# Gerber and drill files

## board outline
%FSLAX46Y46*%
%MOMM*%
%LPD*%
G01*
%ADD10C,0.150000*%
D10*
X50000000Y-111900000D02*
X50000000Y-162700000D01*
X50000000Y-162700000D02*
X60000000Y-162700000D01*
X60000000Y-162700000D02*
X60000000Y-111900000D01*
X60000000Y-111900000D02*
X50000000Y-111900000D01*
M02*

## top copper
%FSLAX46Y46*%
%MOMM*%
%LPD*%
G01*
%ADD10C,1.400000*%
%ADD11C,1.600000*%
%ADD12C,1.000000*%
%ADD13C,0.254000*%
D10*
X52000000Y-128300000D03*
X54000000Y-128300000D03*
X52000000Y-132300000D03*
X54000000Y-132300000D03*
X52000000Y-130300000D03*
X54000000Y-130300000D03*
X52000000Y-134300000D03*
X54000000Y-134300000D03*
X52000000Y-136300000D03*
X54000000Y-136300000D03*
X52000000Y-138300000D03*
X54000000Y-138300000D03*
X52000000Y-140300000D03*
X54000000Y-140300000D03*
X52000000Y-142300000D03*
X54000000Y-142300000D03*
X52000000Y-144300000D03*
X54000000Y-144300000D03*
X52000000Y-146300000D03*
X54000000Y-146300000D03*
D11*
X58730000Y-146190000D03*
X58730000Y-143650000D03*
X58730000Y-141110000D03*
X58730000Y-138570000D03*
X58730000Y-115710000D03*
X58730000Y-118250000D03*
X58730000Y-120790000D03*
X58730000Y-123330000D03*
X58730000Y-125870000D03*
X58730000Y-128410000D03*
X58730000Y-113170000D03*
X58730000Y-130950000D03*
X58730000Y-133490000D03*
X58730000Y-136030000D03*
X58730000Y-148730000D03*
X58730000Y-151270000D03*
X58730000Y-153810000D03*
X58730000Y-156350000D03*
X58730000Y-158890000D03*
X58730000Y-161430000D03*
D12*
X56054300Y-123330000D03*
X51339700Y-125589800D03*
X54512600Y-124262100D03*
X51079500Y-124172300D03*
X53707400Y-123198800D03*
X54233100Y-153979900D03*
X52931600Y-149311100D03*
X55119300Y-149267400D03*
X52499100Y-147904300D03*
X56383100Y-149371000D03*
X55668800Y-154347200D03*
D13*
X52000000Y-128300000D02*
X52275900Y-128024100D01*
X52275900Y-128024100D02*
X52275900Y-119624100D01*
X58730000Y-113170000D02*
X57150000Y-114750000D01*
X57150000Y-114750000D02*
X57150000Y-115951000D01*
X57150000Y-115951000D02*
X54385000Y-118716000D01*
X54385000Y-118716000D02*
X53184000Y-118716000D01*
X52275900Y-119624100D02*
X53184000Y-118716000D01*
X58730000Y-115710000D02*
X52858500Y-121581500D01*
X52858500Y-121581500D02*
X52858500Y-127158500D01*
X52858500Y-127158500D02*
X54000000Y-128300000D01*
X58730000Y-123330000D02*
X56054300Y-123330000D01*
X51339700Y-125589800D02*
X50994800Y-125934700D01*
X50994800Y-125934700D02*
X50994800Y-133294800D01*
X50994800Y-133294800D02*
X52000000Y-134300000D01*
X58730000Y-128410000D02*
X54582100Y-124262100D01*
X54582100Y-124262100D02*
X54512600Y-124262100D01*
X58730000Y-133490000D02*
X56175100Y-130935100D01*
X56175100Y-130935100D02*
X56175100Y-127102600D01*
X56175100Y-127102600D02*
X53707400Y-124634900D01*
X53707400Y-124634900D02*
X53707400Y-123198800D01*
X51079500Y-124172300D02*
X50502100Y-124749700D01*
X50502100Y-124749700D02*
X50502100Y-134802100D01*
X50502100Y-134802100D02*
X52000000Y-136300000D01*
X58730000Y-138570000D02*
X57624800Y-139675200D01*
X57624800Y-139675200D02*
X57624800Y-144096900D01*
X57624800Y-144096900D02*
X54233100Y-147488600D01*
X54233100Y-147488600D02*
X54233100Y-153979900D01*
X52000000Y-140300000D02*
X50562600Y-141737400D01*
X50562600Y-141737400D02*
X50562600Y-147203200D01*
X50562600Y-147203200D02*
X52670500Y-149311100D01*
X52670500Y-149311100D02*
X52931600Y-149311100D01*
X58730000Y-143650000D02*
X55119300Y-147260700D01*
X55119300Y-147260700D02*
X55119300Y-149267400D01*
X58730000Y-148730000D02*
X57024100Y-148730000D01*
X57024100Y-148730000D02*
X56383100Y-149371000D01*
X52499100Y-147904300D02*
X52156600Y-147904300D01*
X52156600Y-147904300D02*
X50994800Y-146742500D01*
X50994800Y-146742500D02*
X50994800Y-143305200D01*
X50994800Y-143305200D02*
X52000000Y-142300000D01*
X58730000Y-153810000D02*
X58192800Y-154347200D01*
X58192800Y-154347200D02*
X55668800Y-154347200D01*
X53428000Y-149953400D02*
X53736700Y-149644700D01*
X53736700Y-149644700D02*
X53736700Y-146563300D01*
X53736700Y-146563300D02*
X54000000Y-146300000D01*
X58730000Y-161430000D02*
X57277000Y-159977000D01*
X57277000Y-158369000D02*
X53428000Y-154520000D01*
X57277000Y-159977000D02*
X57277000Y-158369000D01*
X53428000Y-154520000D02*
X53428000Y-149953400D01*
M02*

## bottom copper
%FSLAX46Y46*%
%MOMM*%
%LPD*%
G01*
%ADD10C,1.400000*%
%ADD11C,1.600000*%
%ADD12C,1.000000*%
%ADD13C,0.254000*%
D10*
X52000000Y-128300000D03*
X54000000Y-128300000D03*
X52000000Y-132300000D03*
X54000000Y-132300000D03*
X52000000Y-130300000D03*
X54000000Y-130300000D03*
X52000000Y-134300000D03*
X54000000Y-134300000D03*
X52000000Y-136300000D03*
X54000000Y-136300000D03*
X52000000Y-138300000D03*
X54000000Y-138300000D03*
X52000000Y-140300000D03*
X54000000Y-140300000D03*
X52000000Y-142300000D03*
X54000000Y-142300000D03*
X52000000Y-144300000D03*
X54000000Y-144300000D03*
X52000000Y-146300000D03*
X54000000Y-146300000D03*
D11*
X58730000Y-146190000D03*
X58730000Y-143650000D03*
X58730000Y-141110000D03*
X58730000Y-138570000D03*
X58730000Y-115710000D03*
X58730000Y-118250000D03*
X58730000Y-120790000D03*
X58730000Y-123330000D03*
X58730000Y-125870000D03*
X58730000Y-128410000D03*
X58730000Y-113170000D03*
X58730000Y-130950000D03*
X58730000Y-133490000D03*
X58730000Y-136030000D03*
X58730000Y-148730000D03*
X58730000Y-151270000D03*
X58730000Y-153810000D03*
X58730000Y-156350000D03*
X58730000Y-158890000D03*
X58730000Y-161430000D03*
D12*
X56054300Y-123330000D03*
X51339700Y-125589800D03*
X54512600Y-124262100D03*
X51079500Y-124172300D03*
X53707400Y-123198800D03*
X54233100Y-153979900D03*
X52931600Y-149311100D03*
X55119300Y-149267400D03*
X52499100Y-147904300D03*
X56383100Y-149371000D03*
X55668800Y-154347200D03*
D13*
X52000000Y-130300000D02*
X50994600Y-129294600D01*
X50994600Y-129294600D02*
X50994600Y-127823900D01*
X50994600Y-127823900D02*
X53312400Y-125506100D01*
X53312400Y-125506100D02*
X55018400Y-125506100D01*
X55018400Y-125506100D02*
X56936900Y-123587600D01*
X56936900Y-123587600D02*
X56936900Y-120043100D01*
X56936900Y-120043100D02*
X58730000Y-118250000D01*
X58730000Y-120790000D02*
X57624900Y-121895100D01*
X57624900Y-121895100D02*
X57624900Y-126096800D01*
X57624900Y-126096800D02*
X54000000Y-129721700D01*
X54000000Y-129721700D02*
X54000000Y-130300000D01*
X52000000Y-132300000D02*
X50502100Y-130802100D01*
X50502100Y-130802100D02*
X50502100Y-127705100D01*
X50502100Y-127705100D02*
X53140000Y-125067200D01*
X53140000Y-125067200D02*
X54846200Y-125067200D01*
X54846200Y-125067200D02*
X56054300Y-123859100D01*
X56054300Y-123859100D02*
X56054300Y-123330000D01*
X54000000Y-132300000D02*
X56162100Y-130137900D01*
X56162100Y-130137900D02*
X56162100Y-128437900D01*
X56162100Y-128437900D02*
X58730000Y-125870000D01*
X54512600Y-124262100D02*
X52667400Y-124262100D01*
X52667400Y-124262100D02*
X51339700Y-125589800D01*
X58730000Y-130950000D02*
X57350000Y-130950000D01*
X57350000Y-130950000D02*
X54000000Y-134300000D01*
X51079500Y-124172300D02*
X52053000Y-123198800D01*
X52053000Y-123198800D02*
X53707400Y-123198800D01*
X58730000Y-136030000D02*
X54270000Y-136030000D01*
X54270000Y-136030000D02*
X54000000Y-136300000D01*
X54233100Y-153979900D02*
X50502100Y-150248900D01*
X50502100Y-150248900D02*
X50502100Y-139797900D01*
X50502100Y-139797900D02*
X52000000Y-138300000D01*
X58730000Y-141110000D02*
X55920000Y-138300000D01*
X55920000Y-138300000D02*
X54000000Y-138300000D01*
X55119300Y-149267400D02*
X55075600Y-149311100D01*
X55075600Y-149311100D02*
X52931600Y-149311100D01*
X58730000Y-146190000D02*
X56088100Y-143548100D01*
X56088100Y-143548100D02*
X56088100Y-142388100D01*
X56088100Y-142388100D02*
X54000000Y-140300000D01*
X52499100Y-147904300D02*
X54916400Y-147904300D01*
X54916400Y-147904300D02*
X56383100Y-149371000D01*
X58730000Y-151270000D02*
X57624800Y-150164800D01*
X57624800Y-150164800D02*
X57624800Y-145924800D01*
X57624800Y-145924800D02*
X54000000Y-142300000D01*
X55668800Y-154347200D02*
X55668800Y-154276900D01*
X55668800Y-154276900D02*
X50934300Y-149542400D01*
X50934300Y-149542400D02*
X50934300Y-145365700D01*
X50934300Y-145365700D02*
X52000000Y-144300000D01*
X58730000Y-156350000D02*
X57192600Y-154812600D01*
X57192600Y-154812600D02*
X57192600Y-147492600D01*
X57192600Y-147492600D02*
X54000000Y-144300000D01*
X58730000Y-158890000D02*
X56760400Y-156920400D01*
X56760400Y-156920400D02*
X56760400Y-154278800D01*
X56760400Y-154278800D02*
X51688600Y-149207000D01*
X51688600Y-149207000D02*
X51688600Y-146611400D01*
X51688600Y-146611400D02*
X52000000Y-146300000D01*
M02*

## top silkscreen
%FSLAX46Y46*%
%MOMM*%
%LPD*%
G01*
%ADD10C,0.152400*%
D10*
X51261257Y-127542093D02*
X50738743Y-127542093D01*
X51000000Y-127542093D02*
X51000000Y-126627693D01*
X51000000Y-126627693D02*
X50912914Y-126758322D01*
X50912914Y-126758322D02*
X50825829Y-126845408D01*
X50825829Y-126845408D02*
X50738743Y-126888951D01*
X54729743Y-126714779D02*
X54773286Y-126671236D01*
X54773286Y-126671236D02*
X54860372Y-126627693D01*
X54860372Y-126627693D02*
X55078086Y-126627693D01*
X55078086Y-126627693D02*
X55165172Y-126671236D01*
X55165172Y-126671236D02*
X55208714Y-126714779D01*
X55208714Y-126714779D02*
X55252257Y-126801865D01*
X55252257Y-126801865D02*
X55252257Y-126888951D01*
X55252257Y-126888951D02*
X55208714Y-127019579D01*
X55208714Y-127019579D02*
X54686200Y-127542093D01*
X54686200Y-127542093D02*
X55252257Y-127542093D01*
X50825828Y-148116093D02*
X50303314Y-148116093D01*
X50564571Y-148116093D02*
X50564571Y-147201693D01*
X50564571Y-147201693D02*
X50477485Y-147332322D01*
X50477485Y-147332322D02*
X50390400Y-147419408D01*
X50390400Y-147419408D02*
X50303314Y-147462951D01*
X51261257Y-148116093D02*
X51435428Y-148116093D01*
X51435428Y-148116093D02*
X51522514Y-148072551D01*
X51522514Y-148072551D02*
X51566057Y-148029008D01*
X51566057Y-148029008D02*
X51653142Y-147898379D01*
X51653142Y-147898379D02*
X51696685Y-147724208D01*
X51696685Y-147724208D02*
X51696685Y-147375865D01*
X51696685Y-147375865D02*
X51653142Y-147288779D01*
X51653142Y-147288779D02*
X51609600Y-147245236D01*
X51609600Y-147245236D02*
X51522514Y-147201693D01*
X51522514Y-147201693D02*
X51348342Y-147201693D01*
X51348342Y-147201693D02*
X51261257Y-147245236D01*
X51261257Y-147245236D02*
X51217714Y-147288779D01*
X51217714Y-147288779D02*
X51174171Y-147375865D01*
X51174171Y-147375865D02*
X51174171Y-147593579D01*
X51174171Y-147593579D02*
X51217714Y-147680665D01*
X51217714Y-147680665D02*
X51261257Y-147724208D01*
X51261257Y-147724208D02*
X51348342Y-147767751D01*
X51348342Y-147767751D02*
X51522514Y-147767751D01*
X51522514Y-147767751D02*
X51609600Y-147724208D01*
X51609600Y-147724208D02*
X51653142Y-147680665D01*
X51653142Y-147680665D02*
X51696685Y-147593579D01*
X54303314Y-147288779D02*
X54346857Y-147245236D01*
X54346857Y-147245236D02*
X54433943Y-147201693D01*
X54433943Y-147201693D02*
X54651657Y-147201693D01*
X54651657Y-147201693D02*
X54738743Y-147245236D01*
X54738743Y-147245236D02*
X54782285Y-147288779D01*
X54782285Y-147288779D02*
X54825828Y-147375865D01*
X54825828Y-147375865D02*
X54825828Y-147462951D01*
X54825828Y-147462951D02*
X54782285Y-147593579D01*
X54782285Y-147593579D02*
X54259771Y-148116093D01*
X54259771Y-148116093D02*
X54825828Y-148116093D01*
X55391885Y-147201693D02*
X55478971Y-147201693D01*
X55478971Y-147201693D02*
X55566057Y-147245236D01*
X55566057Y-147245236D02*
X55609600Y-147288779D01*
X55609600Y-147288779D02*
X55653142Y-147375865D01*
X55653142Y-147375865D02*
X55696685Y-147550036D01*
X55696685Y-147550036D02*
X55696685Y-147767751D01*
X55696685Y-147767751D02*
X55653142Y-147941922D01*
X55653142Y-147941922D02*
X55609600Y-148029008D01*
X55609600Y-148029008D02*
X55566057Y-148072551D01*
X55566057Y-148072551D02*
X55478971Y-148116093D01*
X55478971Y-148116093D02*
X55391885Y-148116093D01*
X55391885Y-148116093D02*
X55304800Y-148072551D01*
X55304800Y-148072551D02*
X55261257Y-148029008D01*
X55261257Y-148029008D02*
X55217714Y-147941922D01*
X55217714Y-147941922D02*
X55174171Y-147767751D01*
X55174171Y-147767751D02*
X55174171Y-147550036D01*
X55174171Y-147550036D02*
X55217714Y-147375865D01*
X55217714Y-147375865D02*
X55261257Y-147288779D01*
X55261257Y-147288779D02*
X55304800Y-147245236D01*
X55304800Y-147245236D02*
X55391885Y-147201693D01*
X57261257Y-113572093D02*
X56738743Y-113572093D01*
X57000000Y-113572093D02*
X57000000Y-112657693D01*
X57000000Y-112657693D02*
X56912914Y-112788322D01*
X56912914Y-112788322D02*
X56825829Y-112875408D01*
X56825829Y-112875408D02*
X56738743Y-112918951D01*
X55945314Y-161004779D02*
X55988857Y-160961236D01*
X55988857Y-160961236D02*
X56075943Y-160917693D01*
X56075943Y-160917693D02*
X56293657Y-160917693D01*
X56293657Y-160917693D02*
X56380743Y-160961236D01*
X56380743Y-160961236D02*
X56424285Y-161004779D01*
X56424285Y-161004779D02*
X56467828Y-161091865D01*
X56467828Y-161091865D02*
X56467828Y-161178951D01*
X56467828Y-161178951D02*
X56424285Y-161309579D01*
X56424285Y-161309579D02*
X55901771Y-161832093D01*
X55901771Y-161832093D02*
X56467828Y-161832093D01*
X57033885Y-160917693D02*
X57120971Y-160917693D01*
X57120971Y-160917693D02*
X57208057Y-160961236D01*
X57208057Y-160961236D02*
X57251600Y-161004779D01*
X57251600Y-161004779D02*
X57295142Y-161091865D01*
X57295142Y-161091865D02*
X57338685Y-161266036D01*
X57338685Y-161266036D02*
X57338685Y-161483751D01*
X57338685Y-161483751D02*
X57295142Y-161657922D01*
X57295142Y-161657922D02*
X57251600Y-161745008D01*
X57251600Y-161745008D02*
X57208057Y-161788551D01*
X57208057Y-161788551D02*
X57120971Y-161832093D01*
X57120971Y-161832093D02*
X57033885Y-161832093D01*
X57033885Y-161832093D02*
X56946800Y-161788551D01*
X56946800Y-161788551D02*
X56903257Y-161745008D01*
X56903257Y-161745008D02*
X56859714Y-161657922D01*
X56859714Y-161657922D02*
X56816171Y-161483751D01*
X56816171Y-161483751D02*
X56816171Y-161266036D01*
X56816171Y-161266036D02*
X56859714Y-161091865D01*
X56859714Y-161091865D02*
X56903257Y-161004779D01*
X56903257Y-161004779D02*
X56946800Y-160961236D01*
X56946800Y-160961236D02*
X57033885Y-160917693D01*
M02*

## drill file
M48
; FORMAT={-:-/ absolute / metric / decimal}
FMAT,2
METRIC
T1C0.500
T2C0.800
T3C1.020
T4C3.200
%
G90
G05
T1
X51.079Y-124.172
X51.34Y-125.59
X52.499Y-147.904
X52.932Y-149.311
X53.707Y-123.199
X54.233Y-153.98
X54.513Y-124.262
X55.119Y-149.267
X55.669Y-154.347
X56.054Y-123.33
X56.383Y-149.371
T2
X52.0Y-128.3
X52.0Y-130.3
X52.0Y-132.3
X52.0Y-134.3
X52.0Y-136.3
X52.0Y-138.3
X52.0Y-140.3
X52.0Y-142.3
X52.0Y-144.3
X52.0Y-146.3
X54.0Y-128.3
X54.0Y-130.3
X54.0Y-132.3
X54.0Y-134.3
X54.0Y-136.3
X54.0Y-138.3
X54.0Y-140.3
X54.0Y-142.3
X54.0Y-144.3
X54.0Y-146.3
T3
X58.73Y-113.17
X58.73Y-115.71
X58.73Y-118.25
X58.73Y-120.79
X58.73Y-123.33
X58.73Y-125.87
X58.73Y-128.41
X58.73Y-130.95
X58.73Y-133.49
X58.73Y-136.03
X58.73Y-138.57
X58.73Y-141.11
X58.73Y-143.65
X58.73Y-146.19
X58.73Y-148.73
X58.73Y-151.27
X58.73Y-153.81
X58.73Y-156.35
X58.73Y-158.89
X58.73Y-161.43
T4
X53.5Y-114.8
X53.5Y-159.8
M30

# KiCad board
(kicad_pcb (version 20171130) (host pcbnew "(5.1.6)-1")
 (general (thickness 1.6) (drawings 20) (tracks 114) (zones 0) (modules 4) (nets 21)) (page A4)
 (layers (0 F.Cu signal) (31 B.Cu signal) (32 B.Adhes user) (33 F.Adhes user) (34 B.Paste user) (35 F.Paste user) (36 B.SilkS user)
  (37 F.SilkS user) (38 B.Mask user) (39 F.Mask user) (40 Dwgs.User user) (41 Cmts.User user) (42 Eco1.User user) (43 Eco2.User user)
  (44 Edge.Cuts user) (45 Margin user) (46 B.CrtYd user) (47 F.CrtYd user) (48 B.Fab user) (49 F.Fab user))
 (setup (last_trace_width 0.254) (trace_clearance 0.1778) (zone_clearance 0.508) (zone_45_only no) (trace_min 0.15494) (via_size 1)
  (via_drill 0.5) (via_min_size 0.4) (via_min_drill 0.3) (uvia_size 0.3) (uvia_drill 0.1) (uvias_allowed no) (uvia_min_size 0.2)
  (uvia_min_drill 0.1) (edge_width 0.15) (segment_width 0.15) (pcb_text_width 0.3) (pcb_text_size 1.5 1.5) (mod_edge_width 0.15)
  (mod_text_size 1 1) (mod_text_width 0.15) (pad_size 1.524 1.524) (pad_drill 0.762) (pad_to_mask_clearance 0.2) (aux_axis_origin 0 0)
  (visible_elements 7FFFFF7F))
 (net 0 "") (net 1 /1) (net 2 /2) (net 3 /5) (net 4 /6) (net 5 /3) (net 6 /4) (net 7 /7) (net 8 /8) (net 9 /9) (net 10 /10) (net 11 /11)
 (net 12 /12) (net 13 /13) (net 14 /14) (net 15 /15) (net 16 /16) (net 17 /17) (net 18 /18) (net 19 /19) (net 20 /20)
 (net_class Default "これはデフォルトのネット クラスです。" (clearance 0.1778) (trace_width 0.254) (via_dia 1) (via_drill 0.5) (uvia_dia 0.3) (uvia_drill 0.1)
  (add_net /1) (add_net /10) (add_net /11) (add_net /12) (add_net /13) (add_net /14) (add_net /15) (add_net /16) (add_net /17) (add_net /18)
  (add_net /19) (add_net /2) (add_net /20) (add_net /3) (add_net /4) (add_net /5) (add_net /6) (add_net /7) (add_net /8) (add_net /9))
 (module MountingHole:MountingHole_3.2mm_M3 (layer F.Cu) (at 53.5 159.8)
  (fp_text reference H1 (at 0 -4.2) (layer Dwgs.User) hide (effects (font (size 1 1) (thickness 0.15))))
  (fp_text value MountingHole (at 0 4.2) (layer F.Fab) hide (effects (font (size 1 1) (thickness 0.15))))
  (pad 1 np_thru_hole circle (at 0 0) (size 3.2 3.2) (drill 3.2) (layers *.Cu *.Mask)))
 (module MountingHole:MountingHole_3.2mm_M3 (layer F.Cu) (at 53.5 114.8)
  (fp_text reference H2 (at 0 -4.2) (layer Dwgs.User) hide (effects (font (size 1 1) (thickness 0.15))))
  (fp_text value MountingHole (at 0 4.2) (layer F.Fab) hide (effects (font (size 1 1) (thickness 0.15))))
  (pad 1 np_thru_hole circle (at 0 0) (size 3.2 3.2) (drill 3.2) (layers *.Cu *.Mask)))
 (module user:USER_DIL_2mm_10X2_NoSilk (layer F.Cu) (at 53 137.3)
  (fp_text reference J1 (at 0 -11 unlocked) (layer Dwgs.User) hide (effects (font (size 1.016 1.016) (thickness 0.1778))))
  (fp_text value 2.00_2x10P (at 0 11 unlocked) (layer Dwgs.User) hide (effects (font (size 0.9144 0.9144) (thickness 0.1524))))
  (pad 1 thru_hole circle (at -1 -9) (size 1.4 1.4) (drill 0.8) (layers *.Cu *.Mask) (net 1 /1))
  (pad 2 thru_hole circle (at 1 -9) (size 1.4 1.4) (drill 0.8) (layers *.Cu *.Mask) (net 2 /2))
  (pad 5 thru_hole circle (at -1 -5) (size 1.4 1.4) (drill 0.8) (layers *.Cu *.Mask) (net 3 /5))
  (pad 6 thru_hole circle (at 1 -5) (size 1.4 1.4) (drill 0.8) (layers *.Cu *.Mask) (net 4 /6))
  (pad 3 thru_hole circle (at -1 -7) (size 1.4 1.4) (drill 0.8) (layers *.Cu *.Mask) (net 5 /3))
  (pad 4 thru_hole circle (at 1 -7) (size 1.4 1.4) (drill 0.8) (layers *.Cu *.Mask) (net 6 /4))
  (pad 7 thru_hole circle (at -1 -3) (size 1.4 1.4) (drill 0.8) (layers *.Cu *.Mask) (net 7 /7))
  (pad 8 thru_hole circle (at 1 -3) (size 1.4 1.4) (drill 0.8) (layers *.Cu *.Mask) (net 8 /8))
  (pad 9 thru_hole circle (at -1 -1) (size 1.4 1.4) (drill 0.8) (layers *.Cu *.Mask) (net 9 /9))
  (pad 10 thru_hole circle (at 1 -1) (size 1.4 1.4) (drill 0.8) (layers *.Cu *.Mask) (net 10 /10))
  (pad 11 thru_hole circle (at -1 1) (size 1.4 1.4) (drill 0.8) (layers *.Cu *.Mask) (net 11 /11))
  (pad 12 thru_hole circle (at 1 1) (size 1.4 1.4) (drill 0.8) (layers *.Cu *.Mask) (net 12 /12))
  (pad 13 thru_hole circle (at -1 3) (size 1.4 1.4) (drill 0.8) (layers *.Cu *.Mask) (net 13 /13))
  (pad 14 thru_hole circle (at 1 3) (size 1.4 1.4) (drill 0.8) (layers *.Cu *.Mask) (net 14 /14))
  (pad 15 thru_hole circle (at -1 5) (size 1.4 1.4) (drill 0.8) (layers *.Cu *.Mask) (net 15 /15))
  (pad 16 thru_hole circle (at 1 5) (size 1.4 1.4) (drill 0.8) (layers *.Cu *.Mask) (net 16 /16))
  (pad 17 thru_hole circle (at -1 7) (size 1.4 1.4) (drill 0.8) (layers *.Cu *.Mask) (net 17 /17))
  (pad 18 thru_hole circle (at 1 7) (size 1.4 1.4) (drill 0.8) (layers *.Cu *.Mask) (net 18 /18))
  (pad 19 thru_hole circle (at -1 9) (size 1.4 1.4) (drill 0.8) (layers *.Cu *.Mask) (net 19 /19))
  (pad 20 thru_hole circle (at 1 9) (size 1.4 1.4) (drill 0.8) (layers *.Cu *.Mask) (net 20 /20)))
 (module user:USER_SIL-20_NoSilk (layer F.Cu) (at 58.73 137.3 270)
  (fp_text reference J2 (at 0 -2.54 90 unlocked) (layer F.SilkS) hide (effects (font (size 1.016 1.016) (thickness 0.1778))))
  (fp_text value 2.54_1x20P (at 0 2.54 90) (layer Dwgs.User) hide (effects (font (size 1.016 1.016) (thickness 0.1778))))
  (pad 14 thru_hole circle (at 8.89 0 270) (size 1.6 1.6) (drill 1.02) (layers *.Cu *.Mask) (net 14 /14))
  (pad 13 thru_hole circle (at 6.35 0 270) (size 1.6 1.6) (drill 1.02) (layers *.Cu *.Mask) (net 13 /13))
  (pad 12 thru_hole circle (at 3.81 0 270) (size 1.6 1.6) (drill 1.02) (layers *.Cu *.Mask) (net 12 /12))
  (pad 11 thru_hole circle (at 1.27 0 270) (size 1.6 1.6) (drill 1.02) (layers *.Cu *.Mask) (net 11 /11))
  (pad 2 thru_hole circle (at -21.59 0 270) (size 1.6 1.6) (drill 1.02) (layers *.Cu *.Mask) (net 2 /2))
  (pad 3 thru_hole circle (at -19.05 0 270) (size 1.6 1.6) (drill 1.02) (layers *.Cu *.Mask) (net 5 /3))
  (pad 4 thru_hole circle (at -16.51 0 270) (size 1.6 1.6) (drill 1.02) (layers *.Cu *.Mask) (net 6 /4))
  (pad 5 thru_hole circle (at -13.97 0 270) (size 1.6 1.6) (drill 1.02) (layers *.Cu *.Mask) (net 3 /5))
  (pad 6 thru_hole circle (at -11.43 0 270) (size 1.6 1.6) (drill 1.02) (layers *.Cu *.Mask) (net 4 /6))
  (pad 7 thru_hole circle (at -8.89 0 270) (size 1.6 1.6) (drill 1.02) (layers *.Cu *.Mask) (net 7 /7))
  (pad 1 thru_hole circle (at -24.13 0 270) (size 1.6 1.6) (drill 1.02) (layers *.Cu *.Mask) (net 1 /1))
  (pad 8 thru_hole circle (at -6.35 0 270) (size 1.6 1.6) (drill 1.02) (layers *.Cu *.Mask) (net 8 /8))
  (pad 9 thru_hole circle (at -3.81 0 270) (size 1.6 1.6) (drill 1.02) (layers *.Cu *.Mask) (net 9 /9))
  (pad 10 thru_hole circle (at -1.27 0 270) (size 1.6 1.6) (drill 1.02) (layers *.Cu *.Mask) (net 10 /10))
  (pad 15 thru_hole circle (at 11.43 0 270) (size 1.6 1.6) (drill 1.02) (layers *.Cu *.Mask) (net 15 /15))
  (pad 16 thru_hole circle (at 13.97 0 270) (size 1.6 1.6) (drill 1.02) (layers *.Cu *.Mask) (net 16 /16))
  (pad 17 thru_hole circle (at 16.51 0 270) (size 1.6 1.6) (drill 1.02) (layers *.Cu *.Mask) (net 17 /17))
  (pad 18 thru_hole circle (at 19.05 0 270) (size 1.6 1.6) (drill 1.02) (layers *.Cu *.Mask) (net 18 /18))
  (pad 19 thru_hole circle (at 21.59 0 270) (size 1.6 1.6) (drill 1.02) (layers *.Cu *.Mask) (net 19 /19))
  (pad 20 thru_hole circle (at 24.13 0 270) (size 1.6 1.6) (drill 1.02) (layers *.Cu *.Mask) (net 20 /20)))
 (gr_line (start 50 111.9) (end 50 162.7) (angle 90) (layer Edge.Cuts) (width 0.15))
 (gr_line (start 50 162.7) (end 60 162.7) (angle 90) (layer Edge.Cuts) (width 0.15))
 (gr_line (start 60 162.7) (end 60 111.9) (angle 90) (layer Edge.Cuts) (width 0.15))
 (gr_line (start 60 111.9) (end 50 111.9) (angle 90) (layer Edge.Cuts) (width 0.15))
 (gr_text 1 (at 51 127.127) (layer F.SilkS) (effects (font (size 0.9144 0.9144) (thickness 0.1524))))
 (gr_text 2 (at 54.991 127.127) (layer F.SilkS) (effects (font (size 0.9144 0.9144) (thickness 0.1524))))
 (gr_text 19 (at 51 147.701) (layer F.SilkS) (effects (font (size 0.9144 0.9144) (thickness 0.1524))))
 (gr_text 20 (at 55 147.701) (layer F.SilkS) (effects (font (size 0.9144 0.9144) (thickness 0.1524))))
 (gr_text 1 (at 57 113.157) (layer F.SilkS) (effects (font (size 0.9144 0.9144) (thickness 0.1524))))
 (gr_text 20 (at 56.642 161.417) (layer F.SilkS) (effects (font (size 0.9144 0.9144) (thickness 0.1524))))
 (segment (start 52 128.3) (end 52.2759 128.0241) (width 0.254) (layer F.Cu) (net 1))
 (segment (start 52.2759 128.0241) (end 52.2759 119.6241) (width 0.254) (layer F.Cu) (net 1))
 (segment (start 58.73 113.17) (end 57.15 114.75) (width 0.254) (layer F.Cu) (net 1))
 (segment (start 57.15 114.75) (end 57.15 115.951) (width 0.254) (layer F.Cu) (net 1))
 (segment (start 57.15 115.951) (end 54.385 118.716) (width 0.254) (layer F.Cu) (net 1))
 (segment (start 54.385 118.716) (end 53.184 118.716) (width 0.254) (layer F.Cu) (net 1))
 (segment (start 52.2759 119.6241) (end 53.184 118.716) (width 0.254) (layer F.Cu) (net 1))
 (segment (start 58.73 115.71) (end 52.8585 121.5815) (width 0.254) (layer F.Cu) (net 2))
 (segment (start 52.8585 121.5815) (end 52.8585 127.1585) (width 0.254) (layer F.Cu) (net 2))
 (segment (start 52.8585 127.1585) (end 54 128.3) (width 0.254) (layer F.Cu) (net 2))
 (segment (start 52 130.3) (end 50.9946 129.2946) (width 0.254) (layer B.Cu) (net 5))
 (segment (start 50.9946 129.2946) (end 50.9946 127.8239) (width 0.254) (layer B.Cu) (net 5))
 (segment (start 50.9946 127.8239) (end 53.3124 125.5061) (width 0.254) (layer B.Cu) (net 5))
 (segment (start 53.3124 125.5061) (end 55.0184 125.5061) (width 0.254) (layer B.Cu) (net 5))
 (segment (start 55.0184 125.5061) (end 56.9369 123.5876) (width 0.254) (layer B.Cu) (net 5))
 (segment (start 56.9369 123.5876) (end 56.9369 120.0431) (width 0.254) (layer B.Cu) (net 5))
 (segment (start 56.9369 120.0431) (end 58.73 118.25) (width 0.254) (layer B.Cu) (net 5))
 (segment (start 58.73 120.79) (end 57.6249 121.8951) (width 0.254) (layer B.Cu) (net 6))
 (segment (start 57.6249 121.8951) (end 57.6249 126.0968) (width 0.254) (layer B.Cu) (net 6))
 (segment (start 57.6249 126.0968) (end 54 129.7217) (width 0.254) (layer B.Cu) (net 6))
 (segment (start 54 129.7217) (end 54 130.3) (width 0.254) (layer B.Cu) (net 6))
 (segment (start 58.73 123.33) (end 56.0543 123.33) (width 0.254) (layer F.Cu) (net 3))
 (segment (start 52 132.3) (end 50.5021 130.8021) (width 0.254) (layer B.Cu) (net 3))
 (segment (start 50.5021 130.8021) (end 50.5021 127.7051) (width 0.254) (layer B.Cu) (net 3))
 (segment (start 50.5021 127.7051) (end 53.14 125.0672) (width 0.254) (layer B.Cu) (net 3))
 (segment (start 53.14 125.0672) (end 54.8462 125.0672) (width 0.254) (layer B.Cu) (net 3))
 (segment (start 54.8462 125.0672) (end 56.0543 123.8591) (width 0.254) (layer B.Cu) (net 3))
 (segment (start 56.0543 123.8591) (end 56.0543 123.33) (width 0.254) (layer B.Cu) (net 3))
 (via (at 56.0543 123.33) (size 1) (layers F.Cu B.Cu) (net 3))
 (segment (start 54 132.3) (end 56.1621 130.1379) (width 0.254) (layer B.Cu) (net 4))
 (segment (start 56.1621 130.1379) (end 56.1621 128.4379) (width 0.254) (layer B.Cu) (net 4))
 (segment (start 56.1621 128.4379) (end 58.73 125.87) (width 0.254) (layer B.Cu) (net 4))
 (segment (start 51.3397 125.5898) (end 50.9948 125.9347) (width 0.254) (layer F.Cu) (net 7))
 (segment (start 50.9948 125.9347) (end 50.9948 133.2948) (width 0.254) (layer F.Cu) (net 7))
 (segment (start 50.9948 133.2948) (end 52 134.3) (width 0.254) (layer F.Cu) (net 7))
 (segment (start 54.5126 124.2621) (end 52.6674 124.2621) (width 0.254) (layer B.Cu) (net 7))
 (segment (start 52.6674 124.2621) (end 51.3397 125.5898) (width 0.254) (layer B.Cu) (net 7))
 (segment (start 58.73 128.41) (end 54.5821 124.2621) (width 0.254) (layer F.Cu) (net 7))
 (segment (start 54.5821 124.2621) (end 54.5126 124.2621) (width 0.254) (layer F.Cu) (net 7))
 (via (at 51.3397 125.5898) (size 1) (layers F.Cu B.Cu) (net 7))
 (via (at 54.5126 124.2621) (size 1) (layers F.Cu B.Cu) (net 7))
 (segment (start 58.73 130.95) (end 57.35 130.95) (width 0.254) (layer B.Cu) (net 8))
 (segment (start 57.35 130.95) (end 54 134.3) (width 0.254) (layer B.Cu) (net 8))
 (segment (start 58.73 133.49) (end 56.1751 130.9351) (width 0.254) (layer F.Cu) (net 9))
 (segment (start 56.1751 130.9351) (end 56.1751 127.1026) (width 0.254) (layer F.Cu) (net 9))
 (segment (start 56.1751 127.1026) (end 53.7074 124.6349) (width 0.254) (layer F.Cu) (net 9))
 (segment (start 53.7074 124.6349) (end 53.7074 123.1988) (width 0.254) (layer F.Cu) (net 9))
 (segment (start 51.0795 124.1723) (end 52.053 123.1988) (width 0.254) (layer B.Cu) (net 9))
 (segment (start 52.053 123.1988) (end 53.7074 123.1988) (width 0.254) (layer B.Cu) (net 9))
 (segment (start 51.0795 124.1723) (end 50.5021 124.7497) (width 0.254) (layer F.Cu) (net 9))
 (segment (start 50.5021 124.7497) (end 50.5021 134.8021) (width 0.254) (layer F.Cu) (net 9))
 (segment (start 50.5021 134.8021) (end 52 136.3) (width 0.254) (layer F.Cu) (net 9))
 (via (at 51.0795 124.1723) (size 1) (layers F.Cu B.Cu) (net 9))
 (via (at 53.7074 123.1988) (size 1) (layers F.Cu B.Cu) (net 9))
 (segment (start 58.73 136.03) (end 54.27 136.03) (width 0.254) (layer B.Cu) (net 10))
 (segment (start 54.27 136.03) (end 54 136.3) (width 0.254) (layer B.Cu) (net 10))
 (segment (start 54.2331 153.9799) (end 50.5021 150.2489) (width 0.254) (layer B.Cu) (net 11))
 (segment (start 50.5021 150.2489) (end 50.5021 139.7979) (width 0.254) (layer B.Cu) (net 11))
 (segment (start 50.5021 139.7979) (end 52 138.3) (width 0.254) (layer B.Cu) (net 11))
 (segment (start 58.73 138.57) (end 57.6248 139.6752) (width 0.254) (layer F.Cu) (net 11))
 (segment (start 57.6248 139.6752) (end 57.6248 144.0969) (width 0.254) (layer F.Cu) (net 11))
 (segment (start 57.6248 144.0969) (end 54.2331 147.4886) (width 0.254) (layer F.Cu) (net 11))
 (segment (start 54.2331 147.4886) (end 54.2331 153.9799) (width 0.254) (layer F.Cu) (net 11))
 (via (at 54.2331 153.9799) (size 1) (layers F.Cu B.Cu) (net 11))
 (segment (start 58.73 141.11) (end 55.92 138.3) (width 0.254) (layer B.Cu) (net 12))
 (segment (start 55.92 138.3) (end 54 138.3) (width 0.254) (layer B.Cu) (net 12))
 (segment (start 55.1193 149.2674) (end 55.0756 149.3111) (width 0.254) (layer B.Cu) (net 13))
 (segment (start 55.0756 149.3111) (end 52.9316 149.3111) (width 0.254) (layer B.Cu) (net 13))
 (segment (start 52 140.3) (end 50.5626 141.7374) (width 0.254) (layer F.Cu) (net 13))
 (segment (start 50.5626 141.7374) (end 50.5626 147.2032) (width 0.254) (layer F.Cu) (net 13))
 (segment (start 50.5626 147.2032) (end 52.6705 149.3111) (width 0.254) (layer F.Cu) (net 13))
 (segment (start 52.6705 149.3111) (end 52.9316 149.3111) (width 0.254) (layer F.Cu) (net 13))
 (segment (start 58.73 143.65) (end 55.1193 147.2607) (width 0.254) (layer F.Cu) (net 13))
 (segment (start 55.1193 147.2607) (end 55.1193 149.2674) (width 0.254) (layer F.Cu) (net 13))
 (via (at 52.9316 149.3111) (size 1) (layers F.Cu B.Cu) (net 13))
 (via (at 55.1193 149.2674) (size 1) (layers F.Cu B.Cu) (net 13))
 (segment (start 58.73 146.19) (end 56.0881 143.5481) (width 0.254) (layer B.Cu) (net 14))
 (segment (start 56.0881 143.5481) (end 56.0881 142.3881) (width 0.254) (layer B.Cu) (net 14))
 (segment (start 56.0881 142.3881) (end 54 140.3) (width 0.254) (layer B.Cu) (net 14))
 (segment (start 58.73 148.73) (end 57.0241 148.73) (width 0.254) (layer F.Cu) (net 15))
 (segment (start 57.0241 148.73) (end 56.3831 149.371) (width 0.254) (layer F.Cu) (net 15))
 (segment (start 52.4991 147.9043) (end 54.9164 147.9043) (width 0.254) (layer B.Cu) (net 15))
 (segment (start 54.9164 147.9043) (end 56.3831 149.371) (width 0.254) (layer B.Cu) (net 15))
 (segment (start 52.4991 147.9043) (end 52.1566 147.9043) (width 0.254) (layer F.Cu) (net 15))
 (segment (start 52.1566 147.9043) (end 50.9948 146.7425) (width 0.254) (layer F.Cu) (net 15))
 (segment (start 50.9948 146.7425) (end 50.9948 143.3052) (width 0.254) (layer F.Cu) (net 15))
 (segment (start 50.9948 143.3052) (end 52 142.3) (width 0.254) (layer F.Cu) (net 15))
 (via (at 52.4991 147.9043) (size 1) (layers F.Cu B.Cu) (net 15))
 (via (at 56.3831 149.371) (size 1) (layers F.Cu B.Cu) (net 15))
 (segment (start 58.73 151.27) (end 57.6248 150.1648) (width 0.254) (layer B.Cu) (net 16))
 (segment (start 57.6248 150.1648) (end 57.6248 145.9248) (width 0.254) (layer B.Cu) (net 16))
 (segment (start 57.6248 145.9248) (end 54 142.3) (width 0.254) (layer B.Cu) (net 16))
 (segment (start 58.73 153.81) (end 58.1928 154.3472) (width 0.254) (layer F.Cu) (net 17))
 (segment (start 58.1928 154.3472) (end 55.6688 154.3472) (width 0.254) (layer F.Cu) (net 17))
 (segment (start 55.6688 154.3472) (end 55.6688 154.2769) (width 0.254) (layer B.Cu) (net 17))
 (segment (start 55.6688 154.2769) (end 50.9343 149.5424) (width 0.254) (layer B.Cu) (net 17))
 (segment (start 50.9343 149.5424) (end 50.9343 145.3657) (width 0.254) (layer B.Cu) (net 17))
 (segment (start 50.9343 145.3657) (end 52 144.3) (width 0.254) (layer B.Cu) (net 17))
 (via (at 55.6688 154.3472) (size 1) (layers F.Cu B.Cu) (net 17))
 (segment (start 58.73 156.35) (end 57.1926 154.8126) (width 0.254) (layer B.Cu) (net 18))
 (segment (start 57.1926 154.8126) (end 57.1926 147.4926) (width 0.254) (layer B.Cu) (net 18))
 (segment (start 57.1926 147.4926) (end 54 144.3) (width 0.254) (layer B.Cu) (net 18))
 (segment (start 58.73 158.89) (end 56.7604 156.9204) (width 0.254) (layer B.Cu) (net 19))
 (segment (start 56.7604 156.9204) (end 56.7604 154.2788) (width 0.254) (layer B.Cu) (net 19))
 (segment (start 56.7604 154.2788) (end 51.6886 149.207) (width 0.254) (layer B.Cu) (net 19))
 (segment (start 51.6886 149.207) (end 51.6886 146.6114) (width 0.254) (layer B.Cu) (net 19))
 (segment (start 51.6886 146.6114) (end 52 146.3) (width 0.254) (layer B.Cu) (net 19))
 (segment (start 53.428 149.9534) (end 53.7367 149.6447) (width 0.254) (layer F.Cu) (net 20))
 (segment (start 53.7367 149.6447) (end 53.7367 146.5633) (width 0.254) (layer F.Cu) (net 20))
 (segment (start 53.7367 146.5633) (end 54 146.3) (width 0.254) (layer F.Cu) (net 20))
 (segment (start 58.73 161.43) (end 57.277 159.977) (width 0.254) (layer F.Cu) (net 20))
 (segment (start 57.277 158.369) (end 53.428 154.52) (width 0.254) (layer F.Cu) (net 20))
 (segment (start 57.277 159.977) (end 57.277 158.369) (width 0.254) (layer F.Cu) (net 20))
 (segment (start 53.428 154.52) (end 53.428 149.9534) (width 0.254) (layer F.Cu) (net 20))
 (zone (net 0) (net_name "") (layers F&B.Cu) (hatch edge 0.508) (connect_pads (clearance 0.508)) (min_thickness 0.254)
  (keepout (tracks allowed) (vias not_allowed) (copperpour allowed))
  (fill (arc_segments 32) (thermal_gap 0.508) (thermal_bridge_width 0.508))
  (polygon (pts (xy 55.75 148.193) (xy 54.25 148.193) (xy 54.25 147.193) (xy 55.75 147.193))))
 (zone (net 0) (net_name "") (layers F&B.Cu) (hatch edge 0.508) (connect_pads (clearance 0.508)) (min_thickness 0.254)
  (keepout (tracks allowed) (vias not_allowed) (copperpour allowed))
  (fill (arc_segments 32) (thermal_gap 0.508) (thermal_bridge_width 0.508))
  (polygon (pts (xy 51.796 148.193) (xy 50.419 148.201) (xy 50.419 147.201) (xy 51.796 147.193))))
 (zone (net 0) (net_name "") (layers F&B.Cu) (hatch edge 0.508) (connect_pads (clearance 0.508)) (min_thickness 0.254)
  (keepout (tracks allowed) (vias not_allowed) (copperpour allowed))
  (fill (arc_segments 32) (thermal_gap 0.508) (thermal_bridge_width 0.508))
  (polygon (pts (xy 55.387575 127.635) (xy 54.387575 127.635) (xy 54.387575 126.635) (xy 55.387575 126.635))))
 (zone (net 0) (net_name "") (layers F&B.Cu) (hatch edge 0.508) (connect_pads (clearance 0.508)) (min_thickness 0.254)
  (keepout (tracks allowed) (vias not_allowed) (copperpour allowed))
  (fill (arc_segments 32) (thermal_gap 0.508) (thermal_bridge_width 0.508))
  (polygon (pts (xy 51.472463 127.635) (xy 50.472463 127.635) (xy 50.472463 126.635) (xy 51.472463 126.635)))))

